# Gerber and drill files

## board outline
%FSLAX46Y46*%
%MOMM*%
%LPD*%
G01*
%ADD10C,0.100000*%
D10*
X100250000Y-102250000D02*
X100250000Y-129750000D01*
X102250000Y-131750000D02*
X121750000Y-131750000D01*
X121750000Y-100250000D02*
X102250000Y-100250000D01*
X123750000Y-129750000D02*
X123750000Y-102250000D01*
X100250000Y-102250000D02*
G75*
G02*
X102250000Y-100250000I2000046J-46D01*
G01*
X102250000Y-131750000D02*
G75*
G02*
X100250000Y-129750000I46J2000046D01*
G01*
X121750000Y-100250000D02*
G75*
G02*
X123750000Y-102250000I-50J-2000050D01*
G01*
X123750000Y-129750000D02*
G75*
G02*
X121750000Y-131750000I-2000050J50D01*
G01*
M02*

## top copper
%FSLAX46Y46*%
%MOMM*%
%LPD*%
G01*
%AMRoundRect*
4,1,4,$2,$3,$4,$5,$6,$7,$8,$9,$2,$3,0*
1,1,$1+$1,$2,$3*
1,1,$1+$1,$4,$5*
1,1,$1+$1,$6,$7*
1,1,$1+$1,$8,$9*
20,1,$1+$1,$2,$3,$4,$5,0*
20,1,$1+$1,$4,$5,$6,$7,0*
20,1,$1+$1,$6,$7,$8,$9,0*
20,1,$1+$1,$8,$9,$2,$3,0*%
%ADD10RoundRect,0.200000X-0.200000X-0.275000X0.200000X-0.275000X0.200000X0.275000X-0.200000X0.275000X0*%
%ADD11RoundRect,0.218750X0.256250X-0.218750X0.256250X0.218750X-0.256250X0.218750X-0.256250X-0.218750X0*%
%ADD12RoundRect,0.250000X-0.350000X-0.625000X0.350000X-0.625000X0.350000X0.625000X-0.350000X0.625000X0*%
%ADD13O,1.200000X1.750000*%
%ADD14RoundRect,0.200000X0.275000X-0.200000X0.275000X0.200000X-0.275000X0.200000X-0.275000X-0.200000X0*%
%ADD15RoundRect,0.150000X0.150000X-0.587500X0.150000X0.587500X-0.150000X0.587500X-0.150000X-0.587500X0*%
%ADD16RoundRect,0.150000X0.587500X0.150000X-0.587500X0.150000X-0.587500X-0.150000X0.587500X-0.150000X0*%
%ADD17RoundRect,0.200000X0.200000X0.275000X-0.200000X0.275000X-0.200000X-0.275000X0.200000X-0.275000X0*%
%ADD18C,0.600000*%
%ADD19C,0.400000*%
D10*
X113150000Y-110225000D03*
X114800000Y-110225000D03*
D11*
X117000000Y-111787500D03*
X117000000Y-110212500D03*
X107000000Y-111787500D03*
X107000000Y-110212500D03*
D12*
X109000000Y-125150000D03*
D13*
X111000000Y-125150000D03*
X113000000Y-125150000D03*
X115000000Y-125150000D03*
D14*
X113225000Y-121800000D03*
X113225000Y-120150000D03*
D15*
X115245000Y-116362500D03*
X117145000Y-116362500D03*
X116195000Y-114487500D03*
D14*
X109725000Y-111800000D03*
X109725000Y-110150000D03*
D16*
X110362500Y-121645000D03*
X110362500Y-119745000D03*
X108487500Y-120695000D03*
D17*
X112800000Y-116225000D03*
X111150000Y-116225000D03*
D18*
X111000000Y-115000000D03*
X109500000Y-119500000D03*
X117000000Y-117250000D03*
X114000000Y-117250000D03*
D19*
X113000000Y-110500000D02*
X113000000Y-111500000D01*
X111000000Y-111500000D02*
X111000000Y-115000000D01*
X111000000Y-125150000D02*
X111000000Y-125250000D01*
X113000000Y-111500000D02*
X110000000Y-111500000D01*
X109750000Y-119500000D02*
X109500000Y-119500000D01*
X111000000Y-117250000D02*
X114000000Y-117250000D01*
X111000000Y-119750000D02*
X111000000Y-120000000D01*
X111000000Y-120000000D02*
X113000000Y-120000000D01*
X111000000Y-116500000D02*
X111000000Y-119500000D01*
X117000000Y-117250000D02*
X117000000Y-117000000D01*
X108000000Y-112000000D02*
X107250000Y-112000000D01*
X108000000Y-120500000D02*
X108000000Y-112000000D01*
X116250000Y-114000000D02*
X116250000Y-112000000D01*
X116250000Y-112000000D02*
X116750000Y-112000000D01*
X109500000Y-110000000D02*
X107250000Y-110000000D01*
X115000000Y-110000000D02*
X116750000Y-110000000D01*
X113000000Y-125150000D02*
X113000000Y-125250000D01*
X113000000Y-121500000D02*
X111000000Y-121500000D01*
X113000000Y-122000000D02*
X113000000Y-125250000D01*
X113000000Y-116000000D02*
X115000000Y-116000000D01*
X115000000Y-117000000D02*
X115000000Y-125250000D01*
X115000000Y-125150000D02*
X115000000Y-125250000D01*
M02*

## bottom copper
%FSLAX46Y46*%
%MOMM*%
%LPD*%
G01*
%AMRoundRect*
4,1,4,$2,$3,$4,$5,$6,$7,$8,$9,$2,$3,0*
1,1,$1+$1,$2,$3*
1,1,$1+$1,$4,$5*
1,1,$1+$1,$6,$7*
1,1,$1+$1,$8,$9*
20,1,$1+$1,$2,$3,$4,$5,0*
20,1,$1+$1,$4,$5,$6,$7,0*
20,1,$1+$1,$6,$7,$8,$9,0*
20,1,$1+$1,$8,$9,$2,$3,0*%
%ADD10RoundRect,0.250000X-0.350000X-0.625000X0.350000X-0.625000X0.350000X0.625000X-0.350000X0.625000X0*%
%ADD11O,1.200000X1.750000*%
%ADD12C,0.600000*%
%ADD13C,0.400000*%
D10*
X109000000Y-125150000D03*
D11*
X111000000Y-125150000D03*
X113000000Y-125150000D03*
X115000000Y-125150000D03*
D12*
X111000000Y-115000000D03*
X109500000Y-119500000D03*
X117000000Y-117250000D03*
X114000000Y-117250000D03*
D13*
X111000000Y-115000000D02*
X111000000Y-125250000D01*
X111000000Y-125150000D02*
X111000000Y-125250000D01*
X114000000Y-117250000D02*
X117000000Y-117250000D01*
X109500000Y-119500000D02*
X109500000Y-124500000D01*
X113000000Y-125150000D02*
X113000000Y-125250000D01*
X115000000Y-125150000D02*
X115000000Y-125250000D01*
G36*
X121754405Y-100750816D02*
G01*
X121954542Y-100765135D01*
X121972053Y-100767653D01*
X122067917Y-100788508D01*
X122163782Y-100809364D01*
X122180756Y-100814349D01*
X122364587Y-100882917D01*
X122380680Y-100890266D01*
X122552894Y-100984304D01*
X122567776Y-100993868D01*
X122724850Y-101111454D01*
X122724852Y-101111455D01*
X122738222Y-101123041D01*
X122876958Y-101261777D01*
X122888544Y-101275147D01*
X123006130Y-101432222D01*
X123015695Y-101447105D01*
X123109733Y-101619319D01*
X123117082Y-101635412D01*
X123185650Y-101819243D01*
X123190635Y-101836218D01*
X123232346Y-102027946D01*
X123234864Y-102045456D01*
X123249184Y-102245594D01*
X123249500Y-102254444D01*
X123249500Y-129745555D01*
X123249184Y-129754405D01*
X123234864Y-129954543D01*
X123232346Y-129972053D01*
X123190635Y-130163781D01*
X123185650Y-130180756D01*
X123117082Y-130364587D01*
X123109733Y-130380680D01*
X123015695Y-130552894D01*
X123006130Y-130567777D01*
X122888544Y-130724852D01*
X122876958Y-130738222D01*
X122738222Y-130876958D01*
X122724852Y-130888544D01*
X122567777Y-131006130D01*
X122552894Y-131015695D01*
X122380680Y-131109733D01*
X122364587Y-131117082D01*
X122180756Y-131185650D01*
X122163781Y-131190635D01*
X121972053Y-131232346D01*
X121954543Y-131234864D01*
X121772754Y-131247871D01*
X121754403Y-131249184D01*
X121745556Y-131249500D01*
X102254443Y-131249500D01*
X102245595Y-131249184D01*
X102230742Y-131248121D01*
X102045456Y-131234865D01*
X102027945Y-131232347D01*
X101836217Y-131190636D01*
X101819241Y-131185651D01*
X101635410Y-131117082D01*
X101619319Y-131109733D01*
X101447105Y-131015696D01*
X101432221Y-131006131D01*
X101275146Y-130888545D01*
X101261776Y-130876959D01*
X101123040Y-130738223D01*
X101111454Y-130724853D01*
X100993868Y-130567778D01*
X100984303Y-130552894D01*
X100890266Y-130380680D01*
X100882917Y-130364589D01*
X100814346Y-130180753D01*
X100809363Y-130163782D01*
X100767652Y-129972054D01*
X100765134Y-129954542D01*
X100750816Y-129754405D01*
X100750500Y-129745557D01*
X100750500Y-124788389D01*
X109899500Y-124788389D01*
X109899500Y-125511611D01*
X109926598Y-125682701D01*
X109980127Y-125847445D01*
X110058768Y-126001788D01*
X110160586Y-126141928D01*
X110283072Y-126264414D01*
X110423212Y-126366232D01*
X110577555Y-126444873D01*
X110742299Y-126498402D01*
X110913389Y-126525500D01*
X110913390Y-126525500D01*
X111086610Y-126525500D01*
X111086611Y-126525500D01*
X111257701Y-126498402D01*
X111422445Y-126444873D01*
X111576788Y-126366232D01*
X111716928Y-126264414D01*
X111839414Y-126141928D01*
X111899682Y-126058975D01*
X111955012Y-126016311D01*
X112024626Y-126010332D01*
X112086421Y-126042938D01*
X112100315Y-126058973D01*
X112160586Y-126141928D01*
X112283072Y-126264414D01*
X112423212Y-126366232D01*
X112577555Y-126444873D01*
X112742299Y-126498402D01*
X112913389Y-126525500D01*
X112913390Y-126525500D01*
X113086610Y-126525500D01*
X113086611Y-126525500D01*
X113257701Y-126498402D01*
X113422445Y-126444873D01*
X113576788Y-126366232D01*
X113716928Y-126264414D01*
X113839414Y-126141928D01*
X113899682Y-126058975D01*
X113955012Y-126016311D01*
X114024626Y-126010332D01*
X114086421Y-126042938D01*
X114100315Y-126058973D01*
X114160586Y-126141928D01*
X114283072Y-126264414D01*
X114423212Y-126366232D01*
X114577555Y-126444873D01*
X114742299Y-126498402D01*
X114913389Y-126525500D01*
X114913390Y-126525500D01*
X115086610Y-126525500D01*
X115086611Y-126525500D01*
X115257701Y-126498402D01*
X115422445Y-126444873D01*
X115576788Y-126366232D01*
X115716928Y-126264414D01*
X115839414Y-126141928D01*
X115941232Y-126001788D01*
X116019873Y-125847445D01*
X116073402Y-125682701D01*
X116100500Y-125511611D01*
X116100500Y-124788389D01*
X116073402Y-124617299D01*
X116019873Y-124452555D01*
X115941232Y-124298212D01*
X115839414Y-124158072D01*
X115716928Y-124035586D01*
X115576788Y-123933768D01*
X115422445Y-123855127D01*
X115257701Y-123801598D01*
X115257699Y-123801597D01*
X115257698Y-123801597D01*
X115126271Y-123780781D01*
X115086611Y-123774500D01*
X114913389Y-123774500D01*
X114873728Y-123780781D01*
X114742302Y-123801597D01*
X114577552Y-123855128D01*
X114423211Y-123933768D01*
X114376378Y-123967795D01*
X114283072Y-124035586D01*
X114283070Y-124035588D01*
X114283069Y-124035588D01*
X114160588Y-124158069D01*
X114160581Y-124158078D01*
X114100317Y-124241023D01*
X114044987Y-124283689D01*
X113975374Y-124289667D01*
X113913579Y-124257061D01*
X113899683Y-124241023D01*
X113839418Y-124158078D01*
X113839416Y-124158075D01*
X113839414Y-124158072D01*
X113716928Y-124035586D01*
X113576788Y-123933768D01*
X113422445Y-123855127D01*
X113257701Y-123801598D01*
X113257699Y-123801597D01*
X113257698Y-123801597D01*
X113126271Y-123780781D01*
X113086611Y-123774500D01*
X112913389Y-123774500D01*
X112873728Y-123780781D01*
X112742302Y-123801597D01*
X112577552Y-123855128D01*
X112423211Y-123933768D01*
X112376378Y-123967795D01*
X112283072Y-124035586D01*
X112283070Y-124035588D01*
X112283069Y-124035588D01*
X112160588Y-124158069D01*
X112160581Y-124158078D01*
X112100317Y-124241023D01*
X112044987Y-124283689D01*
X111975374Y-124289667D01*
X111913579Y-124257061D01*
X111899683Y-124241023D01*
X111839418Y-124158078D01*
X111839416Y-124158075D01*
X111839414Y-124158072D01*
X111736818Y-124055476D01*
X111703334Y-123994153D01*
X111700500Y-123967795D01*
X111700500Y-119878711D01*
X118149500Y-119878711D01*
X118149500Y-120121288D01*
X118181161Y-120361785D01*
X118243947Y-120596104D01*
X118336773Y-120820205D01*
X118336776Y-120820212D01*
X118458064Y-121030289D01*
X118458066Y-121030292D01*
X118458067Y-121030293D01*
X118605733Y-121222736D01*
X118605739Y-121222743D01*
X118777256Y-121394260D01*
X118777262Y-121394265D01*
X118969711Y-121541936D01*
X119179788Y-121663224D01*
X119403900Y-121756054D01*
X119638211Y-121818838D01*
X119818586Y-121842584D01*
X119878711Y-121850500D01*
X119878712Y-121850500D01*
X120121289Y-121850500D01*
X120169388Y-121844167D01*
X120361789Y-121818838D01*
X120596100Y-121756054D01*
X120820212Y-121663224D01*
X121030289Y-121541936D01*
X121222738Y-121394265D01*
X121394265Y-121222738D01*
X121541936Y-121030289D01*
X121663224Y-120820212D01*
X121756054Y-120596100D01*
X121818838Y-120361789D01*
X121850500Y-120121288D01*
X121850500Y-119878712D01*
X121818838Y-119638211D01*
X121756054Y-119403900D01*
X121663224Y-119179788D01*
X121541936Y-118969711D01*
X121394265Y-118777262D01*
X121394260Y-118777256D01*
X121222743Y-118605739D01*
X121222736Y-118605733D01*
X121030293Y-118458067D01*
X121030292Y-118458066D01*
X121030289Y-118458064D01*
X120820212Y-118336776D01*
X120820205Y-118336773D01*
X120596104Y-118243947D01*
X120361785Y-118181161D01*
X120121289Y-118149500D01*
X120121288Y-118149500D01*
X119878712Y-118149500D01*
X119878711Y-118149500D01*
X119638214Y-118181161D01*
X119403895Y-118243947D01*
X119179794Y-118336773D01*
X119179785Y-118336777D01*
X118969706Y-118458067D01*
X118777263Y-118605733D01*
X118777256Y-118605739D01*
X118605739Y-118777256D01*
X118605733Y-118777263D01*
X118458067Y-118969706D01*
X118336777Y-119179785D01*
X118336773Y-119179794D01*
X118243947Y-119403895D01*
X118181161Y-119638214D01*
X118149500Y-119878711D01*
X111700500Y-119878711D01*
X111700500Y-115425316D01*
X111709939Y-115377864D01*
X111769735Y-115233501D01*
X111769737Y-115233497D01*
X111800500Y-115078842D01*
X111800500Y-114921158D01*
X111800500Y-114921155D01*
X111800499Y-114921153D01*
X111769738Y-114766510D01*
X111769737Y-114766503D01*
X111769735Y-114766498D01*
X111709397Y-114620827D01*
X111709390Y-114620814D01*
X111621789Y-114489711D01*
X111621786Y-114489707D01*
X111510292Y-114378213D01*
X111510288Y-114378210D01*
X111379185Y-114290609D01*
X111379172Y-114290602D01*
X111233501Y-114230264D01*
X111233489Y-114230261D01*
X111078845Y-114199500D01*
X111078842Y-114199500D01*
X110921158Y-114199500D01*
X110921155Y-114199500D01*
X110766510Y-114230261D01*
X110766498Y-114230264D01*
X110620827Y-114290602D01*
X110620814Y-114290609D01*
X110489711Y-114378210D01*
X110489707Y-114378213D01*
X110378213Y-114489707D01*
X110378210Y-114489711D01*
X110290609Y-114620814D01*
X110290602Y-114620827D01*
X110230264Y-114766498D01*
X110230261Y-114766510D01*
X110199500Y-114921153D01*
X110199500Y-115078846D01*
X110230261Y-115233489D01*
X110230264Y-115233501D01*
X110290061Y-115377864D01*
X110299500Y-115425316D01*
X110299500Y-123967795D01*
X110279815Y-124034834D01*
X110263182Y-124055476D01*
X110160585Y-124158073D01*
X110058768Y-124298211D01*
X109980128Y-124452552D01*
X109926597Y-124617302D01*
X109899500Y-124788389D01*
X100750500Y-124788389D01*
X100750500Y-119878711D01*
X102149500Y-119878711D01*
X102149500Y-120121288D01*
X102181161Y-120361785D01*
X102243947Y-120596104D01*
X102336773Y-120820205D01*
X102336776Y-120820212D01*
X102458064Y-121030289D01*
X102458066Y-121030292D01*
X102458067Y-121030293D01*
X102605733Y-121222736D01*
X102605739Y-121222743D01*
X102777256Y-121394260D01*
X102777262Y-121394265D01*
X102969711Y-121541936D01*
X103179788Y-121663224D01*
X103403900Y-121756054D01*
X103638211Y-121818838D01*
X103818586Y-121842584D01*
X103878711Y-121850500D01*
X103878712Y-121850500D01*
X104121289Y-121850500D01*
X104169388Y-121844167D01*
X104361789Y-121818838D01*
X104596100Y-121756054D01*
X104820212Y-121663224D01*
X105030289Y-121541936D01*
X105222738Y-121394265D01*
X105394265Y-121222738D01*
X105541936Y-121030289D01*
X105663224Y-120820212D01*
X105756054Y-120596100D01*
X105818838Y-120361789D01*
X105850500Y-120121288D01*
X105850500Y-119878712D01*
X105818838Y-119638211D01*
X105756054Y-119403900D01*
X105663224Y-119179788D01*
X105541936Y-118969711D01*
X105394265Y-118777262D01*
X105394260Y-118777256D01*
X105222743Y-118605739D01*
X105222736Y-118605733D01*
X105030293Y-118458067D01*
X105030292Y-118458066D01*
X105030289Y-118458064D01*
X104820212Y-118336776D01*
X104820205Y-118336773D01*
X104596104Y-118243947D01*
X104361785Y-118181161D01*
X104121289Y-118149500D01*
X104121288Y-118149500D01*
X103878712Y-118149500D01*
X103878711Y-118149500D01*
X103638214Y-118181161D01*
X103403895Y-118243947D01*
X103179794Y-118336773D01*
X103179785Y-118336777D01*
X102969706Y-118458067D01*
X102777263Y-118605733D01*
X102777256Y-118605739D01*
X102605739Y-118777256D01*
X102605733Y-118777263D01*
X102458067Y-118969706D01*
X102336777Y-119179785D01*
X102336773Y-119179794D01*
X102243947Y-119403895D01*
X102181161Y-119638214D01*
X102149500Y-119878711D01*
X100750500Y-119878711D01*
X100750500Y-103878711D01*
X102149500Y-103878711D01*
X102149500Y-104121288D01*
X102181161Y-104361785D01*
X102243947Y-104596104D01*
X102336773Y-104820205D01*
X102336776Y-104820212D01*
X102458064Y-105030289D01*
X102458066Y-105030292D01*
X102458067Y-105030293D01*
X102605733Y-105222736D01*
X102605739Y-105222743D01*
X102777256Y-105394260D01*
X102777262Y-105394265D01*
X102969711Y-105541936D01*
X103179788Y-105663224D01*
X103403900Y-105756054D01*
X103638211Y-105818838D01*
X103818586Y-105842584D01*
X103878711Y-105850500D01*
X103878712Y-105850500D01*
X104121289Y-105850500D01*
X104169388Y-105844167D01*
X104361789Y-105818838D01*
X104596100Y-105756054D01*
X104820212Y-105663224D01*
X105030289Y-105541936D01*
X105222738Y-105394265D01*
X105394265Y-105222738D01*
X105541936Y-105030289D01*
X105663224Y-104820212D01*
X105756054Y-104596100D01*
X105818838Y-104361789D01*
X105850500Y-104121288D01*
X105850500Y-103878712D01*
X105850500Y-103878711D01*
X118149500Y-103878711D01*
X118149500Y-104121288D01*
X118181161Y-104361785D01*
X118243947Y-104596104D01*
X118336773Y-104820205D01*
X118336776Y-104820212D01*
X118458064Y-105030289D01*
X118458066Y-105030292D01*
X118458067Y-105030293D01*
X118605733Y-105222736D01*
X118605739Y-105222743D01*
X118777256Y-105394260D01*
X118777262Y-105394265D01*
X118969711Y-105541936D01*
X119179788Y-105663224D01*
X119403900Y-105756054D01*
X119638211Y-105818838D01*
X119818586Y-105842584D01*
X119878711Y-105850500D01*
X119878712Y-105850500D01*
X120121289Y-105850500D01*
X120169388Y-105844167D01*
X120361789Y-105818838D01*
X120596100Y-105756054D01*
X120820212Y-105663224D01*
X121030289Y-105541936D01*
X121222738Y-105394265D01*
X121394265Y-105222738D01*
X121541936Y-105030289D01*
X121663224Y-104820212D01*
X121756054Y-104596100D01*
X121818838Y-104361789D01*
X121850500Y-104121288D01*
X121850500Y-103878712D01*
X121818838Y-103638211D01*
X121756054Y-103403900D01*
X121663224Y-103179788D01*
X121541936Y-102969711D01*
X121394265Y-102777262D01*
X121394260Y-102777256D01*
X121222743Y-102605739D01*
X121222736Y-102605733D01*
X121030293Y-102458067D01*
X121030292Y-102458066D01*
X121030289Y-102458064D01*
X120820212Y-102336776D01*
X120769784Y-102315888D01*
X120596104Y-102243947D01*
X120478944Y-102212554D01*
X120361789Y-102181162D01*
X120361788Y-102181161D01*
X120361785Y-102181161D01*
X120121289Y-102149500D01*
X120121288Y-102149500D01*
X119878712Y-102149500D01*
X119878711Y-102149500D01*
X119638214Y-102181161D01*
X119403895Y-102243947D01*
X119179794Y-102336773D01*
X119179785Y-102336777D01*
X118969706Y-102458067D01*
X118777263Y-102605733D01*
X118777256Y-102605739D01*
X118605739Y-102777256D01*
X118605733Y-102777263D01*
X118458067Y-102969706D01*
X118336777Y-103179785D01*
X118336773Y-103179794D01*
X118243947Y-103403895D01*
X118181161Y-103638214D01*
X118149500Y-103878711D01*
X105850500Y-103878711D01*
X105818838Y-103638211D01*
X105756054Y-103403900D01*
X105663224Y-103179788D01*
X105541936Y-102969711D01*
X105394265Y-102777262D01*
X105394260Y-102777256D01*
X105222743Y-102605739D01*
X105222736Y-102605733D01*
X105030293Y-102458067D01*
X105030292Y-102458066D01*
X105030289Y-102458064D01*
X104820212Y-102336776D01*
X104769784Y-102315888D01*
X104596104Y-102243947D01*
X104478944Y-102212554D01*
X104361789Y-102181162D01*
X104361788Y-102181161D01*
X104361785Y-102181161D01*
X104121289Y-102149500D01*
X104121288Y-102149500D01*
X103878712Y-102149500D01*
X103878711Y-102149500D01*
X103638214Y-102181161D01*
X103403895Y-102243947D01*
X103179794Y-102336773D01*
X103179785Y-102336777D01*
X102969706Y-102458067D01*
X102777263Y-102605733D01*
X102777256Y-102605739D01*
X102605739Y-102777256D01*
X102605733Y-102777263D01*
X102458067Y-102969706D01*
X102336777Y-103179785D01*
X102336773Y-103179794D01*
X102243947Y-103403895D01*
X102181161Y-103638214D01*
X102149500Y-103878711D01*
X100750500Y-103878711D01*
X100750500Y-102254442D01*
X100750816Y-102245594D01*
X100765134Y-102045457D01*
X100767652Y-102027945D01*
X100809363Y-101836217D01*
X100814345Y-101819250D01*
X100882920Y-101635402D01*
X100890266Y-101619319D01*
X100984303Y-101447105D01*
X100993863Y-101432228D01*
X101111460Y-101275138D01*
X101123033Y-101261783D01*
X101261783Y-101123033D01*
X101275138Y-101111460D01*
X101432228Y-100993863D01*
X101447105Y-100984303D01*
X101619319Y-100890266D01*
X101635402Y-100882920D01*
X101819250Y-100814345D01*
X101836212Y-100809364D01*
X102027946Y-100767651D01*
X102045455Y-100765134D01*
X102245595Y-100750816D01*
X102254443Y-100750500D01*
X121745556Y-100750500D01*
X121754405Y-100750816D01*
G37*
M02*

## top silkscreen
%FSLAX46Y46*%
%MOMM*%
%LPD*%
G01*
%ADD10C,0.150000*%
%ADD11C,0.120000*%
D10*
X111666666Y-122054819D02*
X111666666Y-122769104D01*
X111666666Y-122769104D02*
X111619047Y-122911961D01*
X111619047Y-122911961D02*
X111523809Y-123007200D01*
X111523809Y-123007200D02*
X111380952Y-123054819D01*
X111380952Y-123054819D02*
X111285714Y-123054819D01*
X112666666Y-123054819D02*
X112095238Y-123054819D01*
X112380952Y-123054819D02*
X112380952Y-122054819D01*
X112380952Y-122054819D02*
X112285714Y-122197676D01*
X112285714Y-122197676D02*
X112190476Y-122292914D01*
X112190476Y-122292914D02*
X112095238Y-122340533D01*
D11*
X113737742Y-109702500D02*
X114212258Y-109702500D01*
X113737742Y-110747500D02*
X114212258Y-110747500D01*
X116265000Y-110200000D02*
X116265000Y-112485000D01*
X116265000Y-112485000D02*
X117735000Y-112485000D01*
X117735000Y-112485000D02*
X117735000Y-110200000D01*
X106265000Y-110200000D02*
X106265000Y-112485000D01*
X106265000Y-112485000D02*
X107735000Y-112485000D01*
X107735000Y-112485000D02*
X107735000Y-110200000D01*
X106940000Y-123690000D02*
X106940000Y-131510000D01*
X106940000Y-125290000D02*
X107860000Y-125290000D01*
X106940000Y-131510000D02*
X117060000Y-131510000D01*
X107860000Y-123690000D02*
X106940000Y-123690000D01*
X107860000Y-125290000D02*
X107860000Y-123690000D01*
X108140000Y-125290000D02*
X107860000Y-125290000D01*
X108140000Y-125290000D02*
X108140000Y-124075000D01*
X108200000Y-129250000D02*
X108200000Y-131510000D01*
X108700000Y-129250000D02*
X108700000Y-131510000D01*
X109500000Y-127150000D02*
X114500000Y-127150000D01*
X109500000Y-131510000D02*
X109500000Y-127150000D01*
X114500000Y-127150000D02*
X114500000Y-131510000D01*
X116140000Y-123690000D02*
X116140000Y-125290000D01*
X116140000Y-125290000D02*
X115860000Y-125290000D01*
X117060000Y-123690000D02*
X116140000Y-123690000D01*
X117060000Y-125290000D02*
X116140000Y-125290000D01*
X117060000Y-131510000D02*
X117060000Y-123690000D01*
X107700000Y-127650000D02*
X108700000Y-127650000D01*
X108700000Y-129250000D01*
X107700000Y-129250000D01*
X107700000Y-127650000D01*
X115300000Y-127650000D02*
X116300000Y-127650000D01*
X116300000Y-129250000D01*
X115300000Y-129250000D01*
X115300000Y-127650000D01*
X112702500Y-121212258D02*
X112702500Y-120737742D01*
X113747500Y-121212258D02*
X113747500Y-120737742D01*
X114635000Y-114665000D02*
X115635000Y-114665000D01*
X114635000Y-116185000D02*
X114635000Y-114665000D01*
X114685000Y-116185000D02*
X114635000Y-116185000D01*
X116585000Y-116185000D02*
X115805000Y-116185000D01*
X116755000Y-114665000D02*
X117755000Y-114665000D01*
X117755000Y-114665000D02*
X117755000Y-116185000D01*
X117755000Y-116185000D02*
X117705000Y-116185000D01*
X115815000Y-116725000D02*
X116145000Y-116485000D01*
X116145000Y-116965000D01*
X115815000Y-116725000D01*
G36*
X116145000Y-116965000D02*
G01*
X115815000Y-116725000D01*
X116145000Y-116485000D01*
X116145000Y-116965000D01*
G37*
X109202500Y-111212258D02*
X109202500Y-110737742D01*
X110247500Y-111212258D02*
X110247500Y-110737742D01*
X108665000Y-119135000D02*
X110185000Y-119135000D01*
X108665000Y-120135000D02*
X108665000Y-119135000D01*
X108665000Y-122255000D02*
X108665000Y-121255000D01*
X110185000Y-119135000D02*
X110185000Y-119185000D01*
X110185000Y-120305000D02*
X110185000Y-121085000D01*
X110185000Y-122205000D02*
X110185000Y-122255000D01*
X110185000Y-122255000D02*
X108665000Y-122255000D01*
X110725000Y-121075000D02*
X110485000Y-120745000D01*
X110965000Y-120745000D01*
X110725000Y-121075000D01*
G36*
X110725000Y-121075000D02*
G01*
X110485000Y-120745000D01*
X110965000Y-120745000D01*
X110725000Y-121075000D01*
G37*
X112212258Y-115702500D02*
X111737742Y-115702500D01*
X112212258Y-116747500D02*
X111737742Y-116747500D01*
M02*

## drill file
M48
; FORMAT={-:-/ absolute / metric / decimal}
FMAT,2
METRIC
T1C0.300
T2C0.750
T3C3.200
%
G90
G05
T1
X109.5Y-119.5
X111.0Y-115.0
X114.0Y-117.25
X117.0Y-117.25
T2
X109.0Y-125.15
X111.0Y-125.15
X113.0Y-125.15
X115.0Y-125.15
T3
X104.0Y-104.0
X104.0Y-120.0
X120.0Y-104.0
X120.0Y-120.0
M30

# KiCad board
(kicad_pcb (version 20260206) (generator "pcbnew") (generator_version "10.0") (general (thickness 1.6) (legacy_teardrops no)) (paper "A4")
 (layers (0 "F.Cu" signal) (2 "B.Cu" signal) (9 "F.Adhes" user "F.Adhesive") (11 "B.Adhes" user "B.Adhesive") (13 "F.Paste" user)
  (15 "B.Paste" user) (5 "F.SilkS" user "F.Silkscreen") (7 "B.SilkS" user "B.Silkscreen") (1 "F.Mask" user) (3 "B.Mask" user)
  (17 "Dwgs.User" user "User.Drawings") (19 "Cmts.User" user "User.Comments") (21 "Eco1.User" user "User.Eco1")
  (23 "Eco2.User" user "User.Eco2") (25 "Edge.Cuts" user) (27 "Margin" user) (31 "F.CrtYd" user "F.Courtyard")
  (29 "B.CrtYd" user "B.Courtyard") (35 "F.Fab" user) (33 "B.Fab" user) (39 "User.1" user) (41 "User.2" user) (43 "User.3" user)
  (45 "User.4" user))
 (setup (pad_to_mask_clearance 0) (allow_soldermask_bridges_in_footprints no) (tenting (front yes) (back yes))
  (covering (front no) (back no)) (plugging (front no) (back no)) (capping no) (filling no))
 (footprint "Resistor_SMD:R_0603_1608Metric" (layer "F.Cu") (at 113.975 110.225)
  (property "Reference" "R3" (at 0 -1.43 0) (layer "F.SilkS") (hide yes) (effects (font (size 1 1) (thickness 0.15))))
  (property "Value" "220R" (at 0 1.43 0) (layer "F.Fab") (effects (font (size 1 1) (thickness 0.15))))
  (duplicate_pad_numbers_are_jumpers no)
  (fp_line (start -0.237258 -0.5225) (end 0.237258 -0.5225) (stroke (width 0.12) (type solid)) (layer "F.SilkS"))
  (fp_line (start -0.237258 0.5225) (end 0.237258 0.5225) (stroke (width 0.12) (type solid)) (layer "F.SilkS"))
  (pad "1" smd roundrect (at -0.825 0) (size 0.8 0.95) (layers "F.Cu" "F.Mask" "F.Paste") (roundrect_rratio 0.25) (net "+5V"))
  (pad "2" smd roundrect (at 0.825 0) (size 0.8 0.95) (layers "F.Cu" "F.Mask" "F.Paste") (roundrect_rratio 0.25) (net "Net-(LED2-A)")))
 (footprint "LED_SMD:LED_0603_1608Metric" (layer "F.Cu") (at 117 111 90)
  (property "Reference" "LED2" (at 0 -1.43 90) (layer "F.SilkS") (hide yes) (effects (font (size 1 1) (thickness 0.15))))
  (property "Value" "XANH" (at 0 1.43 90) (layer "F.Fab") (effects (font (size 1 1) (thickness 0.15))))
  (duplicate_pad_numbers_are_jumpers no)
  (fp_line (start 0.8 -0.735) (end -1.485 -0.735) (stroke (width 0.12) (type solid)) (layer "F.SilkS"))
  (fp_line (start -1.485 -0.735) (end -1.485 0.735) (stroke (width 0.12) (type solid)) (layer "F.SilkS"))
  (fp_line (start -1.485 0.735) (end 0.8 0.735) (stroke (width 0.12) (type solid)) (layer "F.SilkS"))
  (pad "1" smd roundrect (at -0.7875 0 90) (size 0.875 0.95) (layers "F.Cu" "F.Mask" "F.Paste") (roundrect_rratio 0.25) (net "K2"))
  (pad "2" smd roundrect (at 0.7875 0 90) (size 0.875 0.95) (layers "F.Cu" "F.Mask" "F.Paste") (roundrect_rratio 0.25) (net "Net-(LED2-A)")))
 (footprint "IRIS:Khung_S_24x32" (layer "F.Cu") (at 100 132)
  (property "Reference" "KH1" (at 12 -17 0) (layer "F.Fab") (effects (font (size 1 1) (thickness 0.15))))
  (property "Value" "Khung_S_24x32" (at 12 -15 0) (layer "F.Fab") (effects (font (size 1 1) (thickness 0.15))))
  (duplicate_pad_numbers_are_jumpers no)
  (fp_line (start 0.25 -29.75) (end 0.25 -2.25) (stroke (width 0.1) (type solid)) (layer "Edge.Cuts"))
  (fp_line (start 2.25 -0.25) (end 21.75 -0.25) (stroke (width 0.1) (type solid)) (layer "Edge.Cuts"))
  (fp_line (start 21.75 -31.75) (end 2.25 -31.75) (stroke (width 0.1) (type solid)) (layer "Edge.Cuts"))
  (fp_line (start 23.75 -2.25) (end 23.75 -29.75) (stroke (width 0.1) (type solid)) (layer "Edge.Cuts"))
  (fp_arc (start 0.25 -29.75) (mid 0.8358 -31.1642) (end 2.25 -31.75) (stroke (width 0.1) (type solid)) (layer "Edge.Cuts"))
  (fp_arc (start 2.25 -0.25) (mid 0.8358 -0.8358) (end 0.25 -2.25) (stroke (width 0.1) (type solid)) (layer "Edge.Cuts"))
  (fp_arc (start 21.75 -31.75) (mid 23.164199 -31.164199) (end 23.75 -29.75) (stroke (width 0.1) (type solid)) (layer "Edge.Cuts"))
  (fp_arc (start 23.75 -2.25) (mid 23.164199 -0.835801) (end 21.75 -0.25) (stroke (width 0.1) (type solid)) (layer "Edge.Cuts"))
  (pad "" np_thru_hole circle (at 4 -28) (size 3.2 3.2) (drill 3.2) (layers "*.Cu" "*.Mask"))
  (pad "" np_thru_hole circle (at 4 -12) (size 3.2 3.2) (drill 3.2) (layers "*.Cu" "*.Mask"))
  (pad "" np_thru_hole circle (at 20 -28) (size 3.2 3.2) (drill 3.2) (layers "*.Cu" "*.Mask"))
  (pad "" np_thru_hole circle (at 20 -12) (size 3.2 3.2) (drill 3.2) (layers "*.Cu" "*.Mask")))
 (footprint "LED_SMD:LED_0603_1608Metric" (layer "F.Cu") (at 107 111 90)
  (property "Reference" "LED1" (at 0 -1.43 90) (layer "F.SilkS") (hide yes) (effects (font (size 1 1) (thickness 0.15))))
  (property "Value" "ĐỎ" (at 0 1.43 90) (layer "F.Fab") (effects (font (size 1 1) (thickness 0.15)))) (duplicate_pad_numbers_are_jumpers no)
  (fp_line (start 0.8 -0.735) (end -1.485 -0.735) (stroke (width 0.12) (type solid)) (layer "F.SilkS"))
  (fp_line (start -1.485 -0.735) (end -1.485 0.735) (stroke (width 0.12) (type solid)) (layer "F.SilkS"))
  (fp_line (start -1.485 0.735) (end 0.8 0.735) (stroke (width 0.12) (type solid)) (layer "F.SilkS"))
  (pad "1" smd roundrect (at -0.7875 0 90) (size 0.875 0.95) (layers "F.Cu" "F.Mask" "F.Paste") (roundrect_rratio 0.25) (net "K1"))
  (pad "2" smd roundrect (at 0.7875 0 90) (size 0.875 0.95) (layers "F.Cu" "F.Mask" "F.Paste") (roundrect_rratio 0.25) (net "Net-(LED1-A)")))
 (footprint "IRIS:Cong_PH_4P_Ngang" (layer "F.Cu") (at 109 125.15)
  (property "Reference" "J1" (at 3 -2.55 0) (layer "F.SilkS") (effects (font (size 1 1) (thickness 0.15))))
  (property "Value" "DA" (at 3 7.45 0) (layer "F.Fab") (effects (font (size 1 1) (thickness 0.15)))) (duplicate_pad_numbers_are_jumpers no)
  (fp_line (start -2.06 -1.46) (end -2.06 6.36) (stroke (width 0.12) (type solid)) (layer "F.SilkS"))
  (fp_line (start -2.06 0.14) (end -1.14 0.14) (stroke (width 0.12) (type solid)) (layer "F.SilkS"))
  (fp_line (start -2.06 6.36) (end 8.06 6.36) (stroke (width 0.12) (type solid)) (layer "F.SilkS"))
  (fp_line (start -1.14 -1.46) (end -2.06 -1.46) (stroke (width 0.12) (type solid)) (layer "F.SilkS"))
  (fp_line (start -1.14 0.14) (end -1.14 -1.46) (stroke (width 0.12) (type solid)) (layer "F.SilkS"))
  (fp_line (start -0.86 0.14) (end -1.14 0.14) (stroke (width 0.12) (type solid)) (layer "F.SilkS"))
  (fp_line (start -0.86 0.14) (end -0.86 -1.075) (stroke (width 0.12) (type solid)) (layer "F.SilkS"))
  (fp_line (start -0.8 4.1) (end -0.8 6.36) (stroke (width 0.12) (type solid)) (layer "F.SilkS"))
  (fp_line (start -0.3 4.1) (end -0.3 6.36) (stroke (width 0.12) (type solid)) (layer "F.SilkS"))
  (fp_line (start 0.5 2) (end 5.5 2) (stroke (width 0.12) (type solid)) (layer "F.SilkS"))
  (fp_line (start 0.5 6.36) (end 0.5 2) (stroke (width 0.12) (type solid)) (layer "F.SilkS"))
  (fp_line (start 5.5 2) (end 5.5 6.36) (stroke (width 0.12) (type solid)) (layer "F.SilkS"))
  (fp_line (start 7.14 -1.46) (end 7.14 0.14) (stroke (width 0.12) (type solid)) (layer "F.SilkS"))
  (fp_line (start 7.14 0.14) (end 6.86 0.14) (stroke (width 0.12) (type solid)) (layer "F.SilkS"))
  (fp_line (start 8.06 -1.46) (end 7.14 -1.46) (stroke (width 0.12) (type solid)) (layer "F.SilkS"))
  (fp_line (start 8.06 0.14) (end 7.14 0.14) (stroke (width 0.12) (type solid)) (layer "F.SilkS"))
  (fp_line (start 8.06 6.36) (end 8.06 -1.46) (stroke (width 0.12) (type solid)) (layer "F.SilkS"))
  (fp_rect (start -1.3 2.5) (end -0.3 4.1) (stroke (width 0.12) (type solid)) (fill no) (layer "F.SilkS"))
  (fp_rect (start 6.3 2.5) (end 7.3 4.1) (stroke (width 0.12) (type solid)) (fill no) (layer "F.SilkS"))
  (pad "1" thru_hole roundrect (at 0 0) (size 1.2 1.75) (drill 0.75) (layers "*.Cu" "*.Mask") (remove_unused_layers no)
   (roundrect_rratio 0.208333) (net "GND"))
  (pad "2" thru_hole oval (at 2 0) (size 1.2 1.75) (drill 0.75) (layers "*.Cu" "*.Mask") (remove_unused_layers no) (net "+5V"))
  (pad "3" thru_hole oval (at 4 0) (size 1.2 1.75) (drill 0.75) (layers "*.Cu" "*.Mask") (remove_unused_layers no) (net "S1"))
  (pad "4" thru_hole oval (at 6 0) (size 1.2 1.75) (drill 0.75) (layers "*.Cu" "*.Mask") (remove_unused_layers no) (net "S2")))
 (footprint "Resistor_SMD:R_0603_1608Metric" (layer "F.Cu") (at 113.225 120.975 90)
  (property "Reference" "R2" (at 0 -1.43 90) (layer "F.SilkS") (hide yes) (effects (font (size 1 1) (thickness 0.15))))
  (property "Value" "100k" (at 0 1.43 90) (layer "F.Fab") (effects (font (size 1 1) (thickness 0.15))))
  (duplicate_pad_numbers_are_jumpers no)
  (fp_line (start -0.237258 -0.5225) (end 0.237258 -0.5225) (stroke (width 0.12) (type solid)) (layer "F.SilkS"))
  (fp_line (start -0.237258 0.5225) (end 0.237258 0.5225) (stroke (width 0.12) (type solid)) (layer "F.SilkS"))
  (pad "1" smd roundrect (at -0.825 0 90) (size 0.8 0.95) (layers "F.Cu" "F.Mask" "F.Paste") (roundrect_rratio 0.25) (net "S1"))
  (pad "2" smd roundrect (at 0.825 0 90) (size 0.8 0.95) (layers "F.Cu" "F.Mask" "F.Paste") (roundrect_rratio 0.25) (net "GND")))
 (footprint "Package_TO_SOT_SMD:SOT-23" (layer "F.Cu") (at 116.195 115.425 90)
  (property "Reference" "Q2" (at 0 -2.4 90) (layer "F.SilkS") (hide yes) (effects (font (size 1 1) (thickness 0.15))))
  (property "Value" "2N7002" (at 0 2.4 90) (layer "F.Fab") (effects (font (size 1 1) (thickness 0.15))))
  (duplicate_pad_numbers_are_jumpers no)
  (fp_line (start 0.76 -1.56) (end 0.76 -0.56) (stroke (width 0.12) (type solid)) (layer "F.SilkS"))
  (fp_line (start -0.76 -1.56) (end 0.76 -1.56) (stroke (width 0.12) (type solid)) (layer "F.SilkS"))
  (fp_line (start -0.76 -1.51) (end -0.76 -1.56) (stroke (width 0.12) (type solid)) (layer "F.SilkS"))
  (fp_line (start -0.76 0.39) (end -0.76 -0.39) (stroke (width 0.12) (type solid)) (layer "F.SilkS"))
  (fp_line (start 0.76 0.56) (end 0.76 1.56) (stroke (width 0.12) (type solid)) (layer "F.SilkS"))
  (fp_line (start 0.76 1.56) (end -0.76 1.56) (stroke (width 0.12) (type solid)) (layer "F.SilkS"))
  (fp_line (start -0.76 1.56) (end -0.76 1.51) (stroke (width 0.12) (type solid)) (layer "F.SilkS"))
  (fp_poly (pts (xy -1.3 -0.38) (xy -1.06 -0.05) (xy -1.54 -0.05)) (stroke (width 0.12) (type solid)) (fill yes) (layer "F.SilkS"))
  (pad "1" smd roundrect (at -0.9375 -0.95 90) (size 1.475 0.6) (layers "F.Cu" "F.Mask" "F.Paste") (roundrect_rratio 0.25) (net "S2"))
  (pad "2" smd roundrect (at -0.9375 0.95 90) (size 1.475 0.6) (layers "F.Cu" "F.Mask" "F.Paste") (roundrect_rratio 0.25) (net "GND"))
  (pad "3" smd roundrect (at 0.9375 0 90) (size 1.475 0.6) (layers "F.Cu" "F.Mask" "F.Paste") (roundrect_rratio 0.25) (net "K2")))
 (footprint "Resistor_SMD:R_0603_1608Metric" (layer "F.Cu") (at 109.725 110.975 90)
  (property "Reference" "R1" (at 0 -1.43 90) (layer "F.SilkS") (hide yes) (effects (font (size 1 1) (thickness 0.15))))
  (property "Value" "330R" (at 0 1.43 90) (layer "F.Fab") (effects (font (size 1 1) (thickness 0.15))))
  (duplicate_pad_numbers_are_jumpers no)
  (fp_line (start -0.237258 -0.5225) (end 0.237258 -0.5225) (stroke (width 0.12) (type solid)) (layer "F.SilkS"))
  (fp_line (start -0.237258 0.5225) (end 0.237258 0.5225) (stroke (width 0.12) (type solid)) (layer "F.SilkS"))
  (pad "1" smd roundrect (at -0.825 0 90) (size 0.8 0.95) (layers "F.Cu" "F.Mask" "F.Paste") (roundrect_rratio 0.25) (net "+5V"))
  (pad "2" smd roundrect (at 0.825 0 90) (size 0.8 0.95) (layers "F.Cu" "F.Mask" "F.Paste") (roundrect_rratio 0.25) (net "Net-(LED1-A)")))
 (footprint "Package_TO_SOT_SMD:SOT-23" (layer "F.Cu") (at 109.425 120.695 180)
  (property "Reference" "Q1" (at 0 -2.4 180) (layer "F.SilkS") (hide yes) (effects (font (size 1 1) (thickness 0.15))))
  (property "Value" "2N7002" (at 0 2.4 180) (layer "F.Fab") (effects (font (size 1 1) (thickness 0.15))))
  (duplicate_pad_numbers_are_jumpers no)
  (fp_line (start 0.76 1.56) (end -0.76 1.56) (stroke (width 0.12) (type solid)) (layer "F.SilkS"))
  (fp_line (start 0.76 0.56) (end 0.76 1.56) (stroke (width 0.12) (type solid)) (layer "F.SilkS"))
  (fp_line (start 0.76 -1.56) (end 0.76 -0.56) (stroke (width 0.12) (type solid)) (layer "F.SilkS"))
  (fp_line (start -0.76 1.56) (end -0.76 1.51) (stroke (width 0.12) (type solid)) (layer "F.SilkS"))
  (fp_line (start -0.76 0.39) (end -0.76 -0.39) (stroke (width 0.12) (type solid)) (layer "F.SilkS"))
  (fp_line (start -0.76 -1.51) (end -0.76 -1.56) (stroke (width 0.12) (type solid)) (layer "F.SilkS"))
  (fp_line (start -0.76 -1.56) (end 0.76 -1.56) (stroke (width 0.12) (type solid)) (layer "F.SilkS"))
  (fp_poly (pts (xy -1.3 -0.38) (xy -1.06 -0.05) (xy -1.54 -0.05)) (stroke (width 0.12) (type solid)) (fill yes) (layer "F.SilkS"))
  (pad "1" smd roundrect (at -0.9375 -0.95 180) (size 1.475 0.6) (layers "F.Cu" "F.Mask" "F.Paste") (roundrect_rratio 0.25) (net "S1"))
  (pad "2" smd roundrect (at -0.9375 0.95 180) (size 1.475 0.6) (layers "F.Cu" "F.Mask" "F.Paste") (roundrect_rratio 0.25) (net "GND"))
  (pad "3" smd roundrect (at 0.9375 0 180) (size 1.475 0.6) (layers "F.Cu" "F.Mask" "F.Paste") (roundrect_rratio 0.25) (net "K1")))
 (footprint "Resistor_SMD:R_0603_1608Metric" (layer "F.Cu") (at 111.975 116.225 180)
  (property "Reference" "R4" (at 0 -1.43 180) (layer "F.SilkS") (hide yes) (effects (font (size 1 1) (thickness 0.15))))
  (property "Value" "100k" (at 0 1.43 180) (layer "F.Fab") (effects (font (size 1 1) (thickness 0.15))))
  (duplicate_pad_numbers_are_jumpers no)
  (fp_line (start -0.237258 0.5225) (end 0.237258 0.5225) (stroke (width 0.12) (type solid)) (layer "F.SilkS"))
  (fp_line (start -0.237258 -0.5225) (end 0.237258 -0.5225) (stroke (width 0.12) (type solid)) (layer "F.SilkS"))
  (pad "1" smd roundrect (at -0.825 0 180) (size 0.8 0.95) (layers "F.Cu" "F.Mask" "F.Paste") (roundrect_rratio 0.25) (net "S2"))
  (pad "2" smd roundrect (at 0.825 0 180) (size 0.8 0.95) (layers "F.Cu" "F.Mask" "F.Paste") (roundrect_rratio 0.25) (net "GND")))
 (segment (start 113 110.5) (end 113 111.5) (width 0.4) (layer "F.Cu") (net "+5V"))
 (segment (start 111 111.5) (end 111 115) (width 0.4) (layer "F.Cu") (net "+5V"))
 (segment (start 111 125.15) (end 111 125.25) (width 0.4) (layer "F.Cu") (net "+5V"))
 (segment (start 113 111.5) (end 110 111.5) (width 0.4) (layer "F.Cu") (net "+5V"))
 (via (at 111 115) (size 0.6) (drill 0.3) (layers "F.Cu" "B.Cu") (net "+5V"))
 (segment (start 111 115) (end 111 125.25) (width 0.4) (layer "B.Cu") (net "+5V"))
 (segment (start 111 125.15) (end 111 125.25) (width 0.4) (layer "B.Cu") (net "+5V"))
 (segment (start 109.75 119.5) (end 109.5 119.5) (width 0.4) (layer "F.Cu") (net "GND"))
 (segment (start 111 117.25) (end 114 117.25) (width 0.4) (layer "F.Cu") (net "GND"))
 (segment (start 111 119.75) (end 111 120) (width 0.4) (layer "F.Cu") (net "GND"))
 (segment (start 111 120) (end 113 120) (width 0.4) (layer "F.Cu") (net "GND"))
 (segment (start 111 116.5) (end 111 119.5) (width 0.4) (layer "F.Cu") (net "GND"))
 (segment (start 117 117.25) (end 117 117) (width 0.4) (layer "F.Cu") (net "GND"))
 (via (at 109.5 119.5) (size 0.6) (drill 0.3) (layers "F.Cu" "B.Cu") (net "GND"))
 (via (at 117 117.25) (size 0.6) (drill 0.3) (layers "F.Cu" "B.Cu") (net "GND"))
 (via (at 114 117.25) (size 0.6) (drill 0.3) (layers "F.Cu" "B.Cu") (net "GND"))
 (segment (start 114 117.25) (end 117 117.25) (width 0.4) (layer "B.Cu") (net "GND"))
 (segment (start 109.5 119.5) (end 109.5 124.5) (width 0.4) (layer "B.Cu") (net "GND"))
 (segment (start 108 112) (end 107.25 112) (width 0.4) (layer "F.Cu") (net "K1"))
 (segment (start 108 120.5) (end 108 112) (width 0.4) (layer "F.Cu") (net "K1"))
 (segment (start 116.25 114) (end 116.25 112) (width 0.4) (layer "F.Cu") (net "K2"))
 (segment (start 116.25 112) (end 116.75 112) (width 0.4) (layer "F.Cu") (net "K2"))
 (segment (start 109.5 110) (end 107.25 110) (width 0.4) (layer "F.Cu") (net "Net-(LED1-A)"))
 (segment (start 115 110) (end 116.75 110) (width 0.4) (layer "F.Cu") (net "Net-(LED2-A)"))
 (segment (start 113 125.15) (end 113 125.25) (width 0.4) (layer "F.Cu") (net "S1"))
 (segment (start 113 121.5) (end 111 121.5) (width 0.4) (layer "F.Cu") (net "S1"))
 (segment (start 113 122) (end 113 125.25) (width 0.4) (layer "F.Cu") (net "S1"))
 (segment (start 113 125.15) (end 113 125.25) (width 0.4) (layer "B.Cu") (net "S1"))
 (segment (start 113 116) (end 115 116) (width 0.4) (layer "F.Cu") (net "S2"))
 (segment (start 115 117) (end 115 125.25) (width 0.4) (layer "F.Cu") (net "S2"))
 (segment (start 115 125.15) (end 115 125.25) (width 0.4) (layer "F.Cu") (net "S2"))
 (segment (start 115 125.15) (end 115 125.25) (width 0.4) (layer "B.Cu") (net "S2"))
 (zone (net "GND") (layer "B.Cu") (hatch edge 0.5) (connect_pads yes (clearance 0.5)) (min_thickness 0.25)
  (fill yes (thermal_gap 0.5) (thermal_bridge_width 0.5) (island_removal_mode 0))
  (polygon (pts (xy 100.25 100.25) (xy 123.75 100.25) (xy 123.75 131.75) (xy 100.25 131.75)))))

